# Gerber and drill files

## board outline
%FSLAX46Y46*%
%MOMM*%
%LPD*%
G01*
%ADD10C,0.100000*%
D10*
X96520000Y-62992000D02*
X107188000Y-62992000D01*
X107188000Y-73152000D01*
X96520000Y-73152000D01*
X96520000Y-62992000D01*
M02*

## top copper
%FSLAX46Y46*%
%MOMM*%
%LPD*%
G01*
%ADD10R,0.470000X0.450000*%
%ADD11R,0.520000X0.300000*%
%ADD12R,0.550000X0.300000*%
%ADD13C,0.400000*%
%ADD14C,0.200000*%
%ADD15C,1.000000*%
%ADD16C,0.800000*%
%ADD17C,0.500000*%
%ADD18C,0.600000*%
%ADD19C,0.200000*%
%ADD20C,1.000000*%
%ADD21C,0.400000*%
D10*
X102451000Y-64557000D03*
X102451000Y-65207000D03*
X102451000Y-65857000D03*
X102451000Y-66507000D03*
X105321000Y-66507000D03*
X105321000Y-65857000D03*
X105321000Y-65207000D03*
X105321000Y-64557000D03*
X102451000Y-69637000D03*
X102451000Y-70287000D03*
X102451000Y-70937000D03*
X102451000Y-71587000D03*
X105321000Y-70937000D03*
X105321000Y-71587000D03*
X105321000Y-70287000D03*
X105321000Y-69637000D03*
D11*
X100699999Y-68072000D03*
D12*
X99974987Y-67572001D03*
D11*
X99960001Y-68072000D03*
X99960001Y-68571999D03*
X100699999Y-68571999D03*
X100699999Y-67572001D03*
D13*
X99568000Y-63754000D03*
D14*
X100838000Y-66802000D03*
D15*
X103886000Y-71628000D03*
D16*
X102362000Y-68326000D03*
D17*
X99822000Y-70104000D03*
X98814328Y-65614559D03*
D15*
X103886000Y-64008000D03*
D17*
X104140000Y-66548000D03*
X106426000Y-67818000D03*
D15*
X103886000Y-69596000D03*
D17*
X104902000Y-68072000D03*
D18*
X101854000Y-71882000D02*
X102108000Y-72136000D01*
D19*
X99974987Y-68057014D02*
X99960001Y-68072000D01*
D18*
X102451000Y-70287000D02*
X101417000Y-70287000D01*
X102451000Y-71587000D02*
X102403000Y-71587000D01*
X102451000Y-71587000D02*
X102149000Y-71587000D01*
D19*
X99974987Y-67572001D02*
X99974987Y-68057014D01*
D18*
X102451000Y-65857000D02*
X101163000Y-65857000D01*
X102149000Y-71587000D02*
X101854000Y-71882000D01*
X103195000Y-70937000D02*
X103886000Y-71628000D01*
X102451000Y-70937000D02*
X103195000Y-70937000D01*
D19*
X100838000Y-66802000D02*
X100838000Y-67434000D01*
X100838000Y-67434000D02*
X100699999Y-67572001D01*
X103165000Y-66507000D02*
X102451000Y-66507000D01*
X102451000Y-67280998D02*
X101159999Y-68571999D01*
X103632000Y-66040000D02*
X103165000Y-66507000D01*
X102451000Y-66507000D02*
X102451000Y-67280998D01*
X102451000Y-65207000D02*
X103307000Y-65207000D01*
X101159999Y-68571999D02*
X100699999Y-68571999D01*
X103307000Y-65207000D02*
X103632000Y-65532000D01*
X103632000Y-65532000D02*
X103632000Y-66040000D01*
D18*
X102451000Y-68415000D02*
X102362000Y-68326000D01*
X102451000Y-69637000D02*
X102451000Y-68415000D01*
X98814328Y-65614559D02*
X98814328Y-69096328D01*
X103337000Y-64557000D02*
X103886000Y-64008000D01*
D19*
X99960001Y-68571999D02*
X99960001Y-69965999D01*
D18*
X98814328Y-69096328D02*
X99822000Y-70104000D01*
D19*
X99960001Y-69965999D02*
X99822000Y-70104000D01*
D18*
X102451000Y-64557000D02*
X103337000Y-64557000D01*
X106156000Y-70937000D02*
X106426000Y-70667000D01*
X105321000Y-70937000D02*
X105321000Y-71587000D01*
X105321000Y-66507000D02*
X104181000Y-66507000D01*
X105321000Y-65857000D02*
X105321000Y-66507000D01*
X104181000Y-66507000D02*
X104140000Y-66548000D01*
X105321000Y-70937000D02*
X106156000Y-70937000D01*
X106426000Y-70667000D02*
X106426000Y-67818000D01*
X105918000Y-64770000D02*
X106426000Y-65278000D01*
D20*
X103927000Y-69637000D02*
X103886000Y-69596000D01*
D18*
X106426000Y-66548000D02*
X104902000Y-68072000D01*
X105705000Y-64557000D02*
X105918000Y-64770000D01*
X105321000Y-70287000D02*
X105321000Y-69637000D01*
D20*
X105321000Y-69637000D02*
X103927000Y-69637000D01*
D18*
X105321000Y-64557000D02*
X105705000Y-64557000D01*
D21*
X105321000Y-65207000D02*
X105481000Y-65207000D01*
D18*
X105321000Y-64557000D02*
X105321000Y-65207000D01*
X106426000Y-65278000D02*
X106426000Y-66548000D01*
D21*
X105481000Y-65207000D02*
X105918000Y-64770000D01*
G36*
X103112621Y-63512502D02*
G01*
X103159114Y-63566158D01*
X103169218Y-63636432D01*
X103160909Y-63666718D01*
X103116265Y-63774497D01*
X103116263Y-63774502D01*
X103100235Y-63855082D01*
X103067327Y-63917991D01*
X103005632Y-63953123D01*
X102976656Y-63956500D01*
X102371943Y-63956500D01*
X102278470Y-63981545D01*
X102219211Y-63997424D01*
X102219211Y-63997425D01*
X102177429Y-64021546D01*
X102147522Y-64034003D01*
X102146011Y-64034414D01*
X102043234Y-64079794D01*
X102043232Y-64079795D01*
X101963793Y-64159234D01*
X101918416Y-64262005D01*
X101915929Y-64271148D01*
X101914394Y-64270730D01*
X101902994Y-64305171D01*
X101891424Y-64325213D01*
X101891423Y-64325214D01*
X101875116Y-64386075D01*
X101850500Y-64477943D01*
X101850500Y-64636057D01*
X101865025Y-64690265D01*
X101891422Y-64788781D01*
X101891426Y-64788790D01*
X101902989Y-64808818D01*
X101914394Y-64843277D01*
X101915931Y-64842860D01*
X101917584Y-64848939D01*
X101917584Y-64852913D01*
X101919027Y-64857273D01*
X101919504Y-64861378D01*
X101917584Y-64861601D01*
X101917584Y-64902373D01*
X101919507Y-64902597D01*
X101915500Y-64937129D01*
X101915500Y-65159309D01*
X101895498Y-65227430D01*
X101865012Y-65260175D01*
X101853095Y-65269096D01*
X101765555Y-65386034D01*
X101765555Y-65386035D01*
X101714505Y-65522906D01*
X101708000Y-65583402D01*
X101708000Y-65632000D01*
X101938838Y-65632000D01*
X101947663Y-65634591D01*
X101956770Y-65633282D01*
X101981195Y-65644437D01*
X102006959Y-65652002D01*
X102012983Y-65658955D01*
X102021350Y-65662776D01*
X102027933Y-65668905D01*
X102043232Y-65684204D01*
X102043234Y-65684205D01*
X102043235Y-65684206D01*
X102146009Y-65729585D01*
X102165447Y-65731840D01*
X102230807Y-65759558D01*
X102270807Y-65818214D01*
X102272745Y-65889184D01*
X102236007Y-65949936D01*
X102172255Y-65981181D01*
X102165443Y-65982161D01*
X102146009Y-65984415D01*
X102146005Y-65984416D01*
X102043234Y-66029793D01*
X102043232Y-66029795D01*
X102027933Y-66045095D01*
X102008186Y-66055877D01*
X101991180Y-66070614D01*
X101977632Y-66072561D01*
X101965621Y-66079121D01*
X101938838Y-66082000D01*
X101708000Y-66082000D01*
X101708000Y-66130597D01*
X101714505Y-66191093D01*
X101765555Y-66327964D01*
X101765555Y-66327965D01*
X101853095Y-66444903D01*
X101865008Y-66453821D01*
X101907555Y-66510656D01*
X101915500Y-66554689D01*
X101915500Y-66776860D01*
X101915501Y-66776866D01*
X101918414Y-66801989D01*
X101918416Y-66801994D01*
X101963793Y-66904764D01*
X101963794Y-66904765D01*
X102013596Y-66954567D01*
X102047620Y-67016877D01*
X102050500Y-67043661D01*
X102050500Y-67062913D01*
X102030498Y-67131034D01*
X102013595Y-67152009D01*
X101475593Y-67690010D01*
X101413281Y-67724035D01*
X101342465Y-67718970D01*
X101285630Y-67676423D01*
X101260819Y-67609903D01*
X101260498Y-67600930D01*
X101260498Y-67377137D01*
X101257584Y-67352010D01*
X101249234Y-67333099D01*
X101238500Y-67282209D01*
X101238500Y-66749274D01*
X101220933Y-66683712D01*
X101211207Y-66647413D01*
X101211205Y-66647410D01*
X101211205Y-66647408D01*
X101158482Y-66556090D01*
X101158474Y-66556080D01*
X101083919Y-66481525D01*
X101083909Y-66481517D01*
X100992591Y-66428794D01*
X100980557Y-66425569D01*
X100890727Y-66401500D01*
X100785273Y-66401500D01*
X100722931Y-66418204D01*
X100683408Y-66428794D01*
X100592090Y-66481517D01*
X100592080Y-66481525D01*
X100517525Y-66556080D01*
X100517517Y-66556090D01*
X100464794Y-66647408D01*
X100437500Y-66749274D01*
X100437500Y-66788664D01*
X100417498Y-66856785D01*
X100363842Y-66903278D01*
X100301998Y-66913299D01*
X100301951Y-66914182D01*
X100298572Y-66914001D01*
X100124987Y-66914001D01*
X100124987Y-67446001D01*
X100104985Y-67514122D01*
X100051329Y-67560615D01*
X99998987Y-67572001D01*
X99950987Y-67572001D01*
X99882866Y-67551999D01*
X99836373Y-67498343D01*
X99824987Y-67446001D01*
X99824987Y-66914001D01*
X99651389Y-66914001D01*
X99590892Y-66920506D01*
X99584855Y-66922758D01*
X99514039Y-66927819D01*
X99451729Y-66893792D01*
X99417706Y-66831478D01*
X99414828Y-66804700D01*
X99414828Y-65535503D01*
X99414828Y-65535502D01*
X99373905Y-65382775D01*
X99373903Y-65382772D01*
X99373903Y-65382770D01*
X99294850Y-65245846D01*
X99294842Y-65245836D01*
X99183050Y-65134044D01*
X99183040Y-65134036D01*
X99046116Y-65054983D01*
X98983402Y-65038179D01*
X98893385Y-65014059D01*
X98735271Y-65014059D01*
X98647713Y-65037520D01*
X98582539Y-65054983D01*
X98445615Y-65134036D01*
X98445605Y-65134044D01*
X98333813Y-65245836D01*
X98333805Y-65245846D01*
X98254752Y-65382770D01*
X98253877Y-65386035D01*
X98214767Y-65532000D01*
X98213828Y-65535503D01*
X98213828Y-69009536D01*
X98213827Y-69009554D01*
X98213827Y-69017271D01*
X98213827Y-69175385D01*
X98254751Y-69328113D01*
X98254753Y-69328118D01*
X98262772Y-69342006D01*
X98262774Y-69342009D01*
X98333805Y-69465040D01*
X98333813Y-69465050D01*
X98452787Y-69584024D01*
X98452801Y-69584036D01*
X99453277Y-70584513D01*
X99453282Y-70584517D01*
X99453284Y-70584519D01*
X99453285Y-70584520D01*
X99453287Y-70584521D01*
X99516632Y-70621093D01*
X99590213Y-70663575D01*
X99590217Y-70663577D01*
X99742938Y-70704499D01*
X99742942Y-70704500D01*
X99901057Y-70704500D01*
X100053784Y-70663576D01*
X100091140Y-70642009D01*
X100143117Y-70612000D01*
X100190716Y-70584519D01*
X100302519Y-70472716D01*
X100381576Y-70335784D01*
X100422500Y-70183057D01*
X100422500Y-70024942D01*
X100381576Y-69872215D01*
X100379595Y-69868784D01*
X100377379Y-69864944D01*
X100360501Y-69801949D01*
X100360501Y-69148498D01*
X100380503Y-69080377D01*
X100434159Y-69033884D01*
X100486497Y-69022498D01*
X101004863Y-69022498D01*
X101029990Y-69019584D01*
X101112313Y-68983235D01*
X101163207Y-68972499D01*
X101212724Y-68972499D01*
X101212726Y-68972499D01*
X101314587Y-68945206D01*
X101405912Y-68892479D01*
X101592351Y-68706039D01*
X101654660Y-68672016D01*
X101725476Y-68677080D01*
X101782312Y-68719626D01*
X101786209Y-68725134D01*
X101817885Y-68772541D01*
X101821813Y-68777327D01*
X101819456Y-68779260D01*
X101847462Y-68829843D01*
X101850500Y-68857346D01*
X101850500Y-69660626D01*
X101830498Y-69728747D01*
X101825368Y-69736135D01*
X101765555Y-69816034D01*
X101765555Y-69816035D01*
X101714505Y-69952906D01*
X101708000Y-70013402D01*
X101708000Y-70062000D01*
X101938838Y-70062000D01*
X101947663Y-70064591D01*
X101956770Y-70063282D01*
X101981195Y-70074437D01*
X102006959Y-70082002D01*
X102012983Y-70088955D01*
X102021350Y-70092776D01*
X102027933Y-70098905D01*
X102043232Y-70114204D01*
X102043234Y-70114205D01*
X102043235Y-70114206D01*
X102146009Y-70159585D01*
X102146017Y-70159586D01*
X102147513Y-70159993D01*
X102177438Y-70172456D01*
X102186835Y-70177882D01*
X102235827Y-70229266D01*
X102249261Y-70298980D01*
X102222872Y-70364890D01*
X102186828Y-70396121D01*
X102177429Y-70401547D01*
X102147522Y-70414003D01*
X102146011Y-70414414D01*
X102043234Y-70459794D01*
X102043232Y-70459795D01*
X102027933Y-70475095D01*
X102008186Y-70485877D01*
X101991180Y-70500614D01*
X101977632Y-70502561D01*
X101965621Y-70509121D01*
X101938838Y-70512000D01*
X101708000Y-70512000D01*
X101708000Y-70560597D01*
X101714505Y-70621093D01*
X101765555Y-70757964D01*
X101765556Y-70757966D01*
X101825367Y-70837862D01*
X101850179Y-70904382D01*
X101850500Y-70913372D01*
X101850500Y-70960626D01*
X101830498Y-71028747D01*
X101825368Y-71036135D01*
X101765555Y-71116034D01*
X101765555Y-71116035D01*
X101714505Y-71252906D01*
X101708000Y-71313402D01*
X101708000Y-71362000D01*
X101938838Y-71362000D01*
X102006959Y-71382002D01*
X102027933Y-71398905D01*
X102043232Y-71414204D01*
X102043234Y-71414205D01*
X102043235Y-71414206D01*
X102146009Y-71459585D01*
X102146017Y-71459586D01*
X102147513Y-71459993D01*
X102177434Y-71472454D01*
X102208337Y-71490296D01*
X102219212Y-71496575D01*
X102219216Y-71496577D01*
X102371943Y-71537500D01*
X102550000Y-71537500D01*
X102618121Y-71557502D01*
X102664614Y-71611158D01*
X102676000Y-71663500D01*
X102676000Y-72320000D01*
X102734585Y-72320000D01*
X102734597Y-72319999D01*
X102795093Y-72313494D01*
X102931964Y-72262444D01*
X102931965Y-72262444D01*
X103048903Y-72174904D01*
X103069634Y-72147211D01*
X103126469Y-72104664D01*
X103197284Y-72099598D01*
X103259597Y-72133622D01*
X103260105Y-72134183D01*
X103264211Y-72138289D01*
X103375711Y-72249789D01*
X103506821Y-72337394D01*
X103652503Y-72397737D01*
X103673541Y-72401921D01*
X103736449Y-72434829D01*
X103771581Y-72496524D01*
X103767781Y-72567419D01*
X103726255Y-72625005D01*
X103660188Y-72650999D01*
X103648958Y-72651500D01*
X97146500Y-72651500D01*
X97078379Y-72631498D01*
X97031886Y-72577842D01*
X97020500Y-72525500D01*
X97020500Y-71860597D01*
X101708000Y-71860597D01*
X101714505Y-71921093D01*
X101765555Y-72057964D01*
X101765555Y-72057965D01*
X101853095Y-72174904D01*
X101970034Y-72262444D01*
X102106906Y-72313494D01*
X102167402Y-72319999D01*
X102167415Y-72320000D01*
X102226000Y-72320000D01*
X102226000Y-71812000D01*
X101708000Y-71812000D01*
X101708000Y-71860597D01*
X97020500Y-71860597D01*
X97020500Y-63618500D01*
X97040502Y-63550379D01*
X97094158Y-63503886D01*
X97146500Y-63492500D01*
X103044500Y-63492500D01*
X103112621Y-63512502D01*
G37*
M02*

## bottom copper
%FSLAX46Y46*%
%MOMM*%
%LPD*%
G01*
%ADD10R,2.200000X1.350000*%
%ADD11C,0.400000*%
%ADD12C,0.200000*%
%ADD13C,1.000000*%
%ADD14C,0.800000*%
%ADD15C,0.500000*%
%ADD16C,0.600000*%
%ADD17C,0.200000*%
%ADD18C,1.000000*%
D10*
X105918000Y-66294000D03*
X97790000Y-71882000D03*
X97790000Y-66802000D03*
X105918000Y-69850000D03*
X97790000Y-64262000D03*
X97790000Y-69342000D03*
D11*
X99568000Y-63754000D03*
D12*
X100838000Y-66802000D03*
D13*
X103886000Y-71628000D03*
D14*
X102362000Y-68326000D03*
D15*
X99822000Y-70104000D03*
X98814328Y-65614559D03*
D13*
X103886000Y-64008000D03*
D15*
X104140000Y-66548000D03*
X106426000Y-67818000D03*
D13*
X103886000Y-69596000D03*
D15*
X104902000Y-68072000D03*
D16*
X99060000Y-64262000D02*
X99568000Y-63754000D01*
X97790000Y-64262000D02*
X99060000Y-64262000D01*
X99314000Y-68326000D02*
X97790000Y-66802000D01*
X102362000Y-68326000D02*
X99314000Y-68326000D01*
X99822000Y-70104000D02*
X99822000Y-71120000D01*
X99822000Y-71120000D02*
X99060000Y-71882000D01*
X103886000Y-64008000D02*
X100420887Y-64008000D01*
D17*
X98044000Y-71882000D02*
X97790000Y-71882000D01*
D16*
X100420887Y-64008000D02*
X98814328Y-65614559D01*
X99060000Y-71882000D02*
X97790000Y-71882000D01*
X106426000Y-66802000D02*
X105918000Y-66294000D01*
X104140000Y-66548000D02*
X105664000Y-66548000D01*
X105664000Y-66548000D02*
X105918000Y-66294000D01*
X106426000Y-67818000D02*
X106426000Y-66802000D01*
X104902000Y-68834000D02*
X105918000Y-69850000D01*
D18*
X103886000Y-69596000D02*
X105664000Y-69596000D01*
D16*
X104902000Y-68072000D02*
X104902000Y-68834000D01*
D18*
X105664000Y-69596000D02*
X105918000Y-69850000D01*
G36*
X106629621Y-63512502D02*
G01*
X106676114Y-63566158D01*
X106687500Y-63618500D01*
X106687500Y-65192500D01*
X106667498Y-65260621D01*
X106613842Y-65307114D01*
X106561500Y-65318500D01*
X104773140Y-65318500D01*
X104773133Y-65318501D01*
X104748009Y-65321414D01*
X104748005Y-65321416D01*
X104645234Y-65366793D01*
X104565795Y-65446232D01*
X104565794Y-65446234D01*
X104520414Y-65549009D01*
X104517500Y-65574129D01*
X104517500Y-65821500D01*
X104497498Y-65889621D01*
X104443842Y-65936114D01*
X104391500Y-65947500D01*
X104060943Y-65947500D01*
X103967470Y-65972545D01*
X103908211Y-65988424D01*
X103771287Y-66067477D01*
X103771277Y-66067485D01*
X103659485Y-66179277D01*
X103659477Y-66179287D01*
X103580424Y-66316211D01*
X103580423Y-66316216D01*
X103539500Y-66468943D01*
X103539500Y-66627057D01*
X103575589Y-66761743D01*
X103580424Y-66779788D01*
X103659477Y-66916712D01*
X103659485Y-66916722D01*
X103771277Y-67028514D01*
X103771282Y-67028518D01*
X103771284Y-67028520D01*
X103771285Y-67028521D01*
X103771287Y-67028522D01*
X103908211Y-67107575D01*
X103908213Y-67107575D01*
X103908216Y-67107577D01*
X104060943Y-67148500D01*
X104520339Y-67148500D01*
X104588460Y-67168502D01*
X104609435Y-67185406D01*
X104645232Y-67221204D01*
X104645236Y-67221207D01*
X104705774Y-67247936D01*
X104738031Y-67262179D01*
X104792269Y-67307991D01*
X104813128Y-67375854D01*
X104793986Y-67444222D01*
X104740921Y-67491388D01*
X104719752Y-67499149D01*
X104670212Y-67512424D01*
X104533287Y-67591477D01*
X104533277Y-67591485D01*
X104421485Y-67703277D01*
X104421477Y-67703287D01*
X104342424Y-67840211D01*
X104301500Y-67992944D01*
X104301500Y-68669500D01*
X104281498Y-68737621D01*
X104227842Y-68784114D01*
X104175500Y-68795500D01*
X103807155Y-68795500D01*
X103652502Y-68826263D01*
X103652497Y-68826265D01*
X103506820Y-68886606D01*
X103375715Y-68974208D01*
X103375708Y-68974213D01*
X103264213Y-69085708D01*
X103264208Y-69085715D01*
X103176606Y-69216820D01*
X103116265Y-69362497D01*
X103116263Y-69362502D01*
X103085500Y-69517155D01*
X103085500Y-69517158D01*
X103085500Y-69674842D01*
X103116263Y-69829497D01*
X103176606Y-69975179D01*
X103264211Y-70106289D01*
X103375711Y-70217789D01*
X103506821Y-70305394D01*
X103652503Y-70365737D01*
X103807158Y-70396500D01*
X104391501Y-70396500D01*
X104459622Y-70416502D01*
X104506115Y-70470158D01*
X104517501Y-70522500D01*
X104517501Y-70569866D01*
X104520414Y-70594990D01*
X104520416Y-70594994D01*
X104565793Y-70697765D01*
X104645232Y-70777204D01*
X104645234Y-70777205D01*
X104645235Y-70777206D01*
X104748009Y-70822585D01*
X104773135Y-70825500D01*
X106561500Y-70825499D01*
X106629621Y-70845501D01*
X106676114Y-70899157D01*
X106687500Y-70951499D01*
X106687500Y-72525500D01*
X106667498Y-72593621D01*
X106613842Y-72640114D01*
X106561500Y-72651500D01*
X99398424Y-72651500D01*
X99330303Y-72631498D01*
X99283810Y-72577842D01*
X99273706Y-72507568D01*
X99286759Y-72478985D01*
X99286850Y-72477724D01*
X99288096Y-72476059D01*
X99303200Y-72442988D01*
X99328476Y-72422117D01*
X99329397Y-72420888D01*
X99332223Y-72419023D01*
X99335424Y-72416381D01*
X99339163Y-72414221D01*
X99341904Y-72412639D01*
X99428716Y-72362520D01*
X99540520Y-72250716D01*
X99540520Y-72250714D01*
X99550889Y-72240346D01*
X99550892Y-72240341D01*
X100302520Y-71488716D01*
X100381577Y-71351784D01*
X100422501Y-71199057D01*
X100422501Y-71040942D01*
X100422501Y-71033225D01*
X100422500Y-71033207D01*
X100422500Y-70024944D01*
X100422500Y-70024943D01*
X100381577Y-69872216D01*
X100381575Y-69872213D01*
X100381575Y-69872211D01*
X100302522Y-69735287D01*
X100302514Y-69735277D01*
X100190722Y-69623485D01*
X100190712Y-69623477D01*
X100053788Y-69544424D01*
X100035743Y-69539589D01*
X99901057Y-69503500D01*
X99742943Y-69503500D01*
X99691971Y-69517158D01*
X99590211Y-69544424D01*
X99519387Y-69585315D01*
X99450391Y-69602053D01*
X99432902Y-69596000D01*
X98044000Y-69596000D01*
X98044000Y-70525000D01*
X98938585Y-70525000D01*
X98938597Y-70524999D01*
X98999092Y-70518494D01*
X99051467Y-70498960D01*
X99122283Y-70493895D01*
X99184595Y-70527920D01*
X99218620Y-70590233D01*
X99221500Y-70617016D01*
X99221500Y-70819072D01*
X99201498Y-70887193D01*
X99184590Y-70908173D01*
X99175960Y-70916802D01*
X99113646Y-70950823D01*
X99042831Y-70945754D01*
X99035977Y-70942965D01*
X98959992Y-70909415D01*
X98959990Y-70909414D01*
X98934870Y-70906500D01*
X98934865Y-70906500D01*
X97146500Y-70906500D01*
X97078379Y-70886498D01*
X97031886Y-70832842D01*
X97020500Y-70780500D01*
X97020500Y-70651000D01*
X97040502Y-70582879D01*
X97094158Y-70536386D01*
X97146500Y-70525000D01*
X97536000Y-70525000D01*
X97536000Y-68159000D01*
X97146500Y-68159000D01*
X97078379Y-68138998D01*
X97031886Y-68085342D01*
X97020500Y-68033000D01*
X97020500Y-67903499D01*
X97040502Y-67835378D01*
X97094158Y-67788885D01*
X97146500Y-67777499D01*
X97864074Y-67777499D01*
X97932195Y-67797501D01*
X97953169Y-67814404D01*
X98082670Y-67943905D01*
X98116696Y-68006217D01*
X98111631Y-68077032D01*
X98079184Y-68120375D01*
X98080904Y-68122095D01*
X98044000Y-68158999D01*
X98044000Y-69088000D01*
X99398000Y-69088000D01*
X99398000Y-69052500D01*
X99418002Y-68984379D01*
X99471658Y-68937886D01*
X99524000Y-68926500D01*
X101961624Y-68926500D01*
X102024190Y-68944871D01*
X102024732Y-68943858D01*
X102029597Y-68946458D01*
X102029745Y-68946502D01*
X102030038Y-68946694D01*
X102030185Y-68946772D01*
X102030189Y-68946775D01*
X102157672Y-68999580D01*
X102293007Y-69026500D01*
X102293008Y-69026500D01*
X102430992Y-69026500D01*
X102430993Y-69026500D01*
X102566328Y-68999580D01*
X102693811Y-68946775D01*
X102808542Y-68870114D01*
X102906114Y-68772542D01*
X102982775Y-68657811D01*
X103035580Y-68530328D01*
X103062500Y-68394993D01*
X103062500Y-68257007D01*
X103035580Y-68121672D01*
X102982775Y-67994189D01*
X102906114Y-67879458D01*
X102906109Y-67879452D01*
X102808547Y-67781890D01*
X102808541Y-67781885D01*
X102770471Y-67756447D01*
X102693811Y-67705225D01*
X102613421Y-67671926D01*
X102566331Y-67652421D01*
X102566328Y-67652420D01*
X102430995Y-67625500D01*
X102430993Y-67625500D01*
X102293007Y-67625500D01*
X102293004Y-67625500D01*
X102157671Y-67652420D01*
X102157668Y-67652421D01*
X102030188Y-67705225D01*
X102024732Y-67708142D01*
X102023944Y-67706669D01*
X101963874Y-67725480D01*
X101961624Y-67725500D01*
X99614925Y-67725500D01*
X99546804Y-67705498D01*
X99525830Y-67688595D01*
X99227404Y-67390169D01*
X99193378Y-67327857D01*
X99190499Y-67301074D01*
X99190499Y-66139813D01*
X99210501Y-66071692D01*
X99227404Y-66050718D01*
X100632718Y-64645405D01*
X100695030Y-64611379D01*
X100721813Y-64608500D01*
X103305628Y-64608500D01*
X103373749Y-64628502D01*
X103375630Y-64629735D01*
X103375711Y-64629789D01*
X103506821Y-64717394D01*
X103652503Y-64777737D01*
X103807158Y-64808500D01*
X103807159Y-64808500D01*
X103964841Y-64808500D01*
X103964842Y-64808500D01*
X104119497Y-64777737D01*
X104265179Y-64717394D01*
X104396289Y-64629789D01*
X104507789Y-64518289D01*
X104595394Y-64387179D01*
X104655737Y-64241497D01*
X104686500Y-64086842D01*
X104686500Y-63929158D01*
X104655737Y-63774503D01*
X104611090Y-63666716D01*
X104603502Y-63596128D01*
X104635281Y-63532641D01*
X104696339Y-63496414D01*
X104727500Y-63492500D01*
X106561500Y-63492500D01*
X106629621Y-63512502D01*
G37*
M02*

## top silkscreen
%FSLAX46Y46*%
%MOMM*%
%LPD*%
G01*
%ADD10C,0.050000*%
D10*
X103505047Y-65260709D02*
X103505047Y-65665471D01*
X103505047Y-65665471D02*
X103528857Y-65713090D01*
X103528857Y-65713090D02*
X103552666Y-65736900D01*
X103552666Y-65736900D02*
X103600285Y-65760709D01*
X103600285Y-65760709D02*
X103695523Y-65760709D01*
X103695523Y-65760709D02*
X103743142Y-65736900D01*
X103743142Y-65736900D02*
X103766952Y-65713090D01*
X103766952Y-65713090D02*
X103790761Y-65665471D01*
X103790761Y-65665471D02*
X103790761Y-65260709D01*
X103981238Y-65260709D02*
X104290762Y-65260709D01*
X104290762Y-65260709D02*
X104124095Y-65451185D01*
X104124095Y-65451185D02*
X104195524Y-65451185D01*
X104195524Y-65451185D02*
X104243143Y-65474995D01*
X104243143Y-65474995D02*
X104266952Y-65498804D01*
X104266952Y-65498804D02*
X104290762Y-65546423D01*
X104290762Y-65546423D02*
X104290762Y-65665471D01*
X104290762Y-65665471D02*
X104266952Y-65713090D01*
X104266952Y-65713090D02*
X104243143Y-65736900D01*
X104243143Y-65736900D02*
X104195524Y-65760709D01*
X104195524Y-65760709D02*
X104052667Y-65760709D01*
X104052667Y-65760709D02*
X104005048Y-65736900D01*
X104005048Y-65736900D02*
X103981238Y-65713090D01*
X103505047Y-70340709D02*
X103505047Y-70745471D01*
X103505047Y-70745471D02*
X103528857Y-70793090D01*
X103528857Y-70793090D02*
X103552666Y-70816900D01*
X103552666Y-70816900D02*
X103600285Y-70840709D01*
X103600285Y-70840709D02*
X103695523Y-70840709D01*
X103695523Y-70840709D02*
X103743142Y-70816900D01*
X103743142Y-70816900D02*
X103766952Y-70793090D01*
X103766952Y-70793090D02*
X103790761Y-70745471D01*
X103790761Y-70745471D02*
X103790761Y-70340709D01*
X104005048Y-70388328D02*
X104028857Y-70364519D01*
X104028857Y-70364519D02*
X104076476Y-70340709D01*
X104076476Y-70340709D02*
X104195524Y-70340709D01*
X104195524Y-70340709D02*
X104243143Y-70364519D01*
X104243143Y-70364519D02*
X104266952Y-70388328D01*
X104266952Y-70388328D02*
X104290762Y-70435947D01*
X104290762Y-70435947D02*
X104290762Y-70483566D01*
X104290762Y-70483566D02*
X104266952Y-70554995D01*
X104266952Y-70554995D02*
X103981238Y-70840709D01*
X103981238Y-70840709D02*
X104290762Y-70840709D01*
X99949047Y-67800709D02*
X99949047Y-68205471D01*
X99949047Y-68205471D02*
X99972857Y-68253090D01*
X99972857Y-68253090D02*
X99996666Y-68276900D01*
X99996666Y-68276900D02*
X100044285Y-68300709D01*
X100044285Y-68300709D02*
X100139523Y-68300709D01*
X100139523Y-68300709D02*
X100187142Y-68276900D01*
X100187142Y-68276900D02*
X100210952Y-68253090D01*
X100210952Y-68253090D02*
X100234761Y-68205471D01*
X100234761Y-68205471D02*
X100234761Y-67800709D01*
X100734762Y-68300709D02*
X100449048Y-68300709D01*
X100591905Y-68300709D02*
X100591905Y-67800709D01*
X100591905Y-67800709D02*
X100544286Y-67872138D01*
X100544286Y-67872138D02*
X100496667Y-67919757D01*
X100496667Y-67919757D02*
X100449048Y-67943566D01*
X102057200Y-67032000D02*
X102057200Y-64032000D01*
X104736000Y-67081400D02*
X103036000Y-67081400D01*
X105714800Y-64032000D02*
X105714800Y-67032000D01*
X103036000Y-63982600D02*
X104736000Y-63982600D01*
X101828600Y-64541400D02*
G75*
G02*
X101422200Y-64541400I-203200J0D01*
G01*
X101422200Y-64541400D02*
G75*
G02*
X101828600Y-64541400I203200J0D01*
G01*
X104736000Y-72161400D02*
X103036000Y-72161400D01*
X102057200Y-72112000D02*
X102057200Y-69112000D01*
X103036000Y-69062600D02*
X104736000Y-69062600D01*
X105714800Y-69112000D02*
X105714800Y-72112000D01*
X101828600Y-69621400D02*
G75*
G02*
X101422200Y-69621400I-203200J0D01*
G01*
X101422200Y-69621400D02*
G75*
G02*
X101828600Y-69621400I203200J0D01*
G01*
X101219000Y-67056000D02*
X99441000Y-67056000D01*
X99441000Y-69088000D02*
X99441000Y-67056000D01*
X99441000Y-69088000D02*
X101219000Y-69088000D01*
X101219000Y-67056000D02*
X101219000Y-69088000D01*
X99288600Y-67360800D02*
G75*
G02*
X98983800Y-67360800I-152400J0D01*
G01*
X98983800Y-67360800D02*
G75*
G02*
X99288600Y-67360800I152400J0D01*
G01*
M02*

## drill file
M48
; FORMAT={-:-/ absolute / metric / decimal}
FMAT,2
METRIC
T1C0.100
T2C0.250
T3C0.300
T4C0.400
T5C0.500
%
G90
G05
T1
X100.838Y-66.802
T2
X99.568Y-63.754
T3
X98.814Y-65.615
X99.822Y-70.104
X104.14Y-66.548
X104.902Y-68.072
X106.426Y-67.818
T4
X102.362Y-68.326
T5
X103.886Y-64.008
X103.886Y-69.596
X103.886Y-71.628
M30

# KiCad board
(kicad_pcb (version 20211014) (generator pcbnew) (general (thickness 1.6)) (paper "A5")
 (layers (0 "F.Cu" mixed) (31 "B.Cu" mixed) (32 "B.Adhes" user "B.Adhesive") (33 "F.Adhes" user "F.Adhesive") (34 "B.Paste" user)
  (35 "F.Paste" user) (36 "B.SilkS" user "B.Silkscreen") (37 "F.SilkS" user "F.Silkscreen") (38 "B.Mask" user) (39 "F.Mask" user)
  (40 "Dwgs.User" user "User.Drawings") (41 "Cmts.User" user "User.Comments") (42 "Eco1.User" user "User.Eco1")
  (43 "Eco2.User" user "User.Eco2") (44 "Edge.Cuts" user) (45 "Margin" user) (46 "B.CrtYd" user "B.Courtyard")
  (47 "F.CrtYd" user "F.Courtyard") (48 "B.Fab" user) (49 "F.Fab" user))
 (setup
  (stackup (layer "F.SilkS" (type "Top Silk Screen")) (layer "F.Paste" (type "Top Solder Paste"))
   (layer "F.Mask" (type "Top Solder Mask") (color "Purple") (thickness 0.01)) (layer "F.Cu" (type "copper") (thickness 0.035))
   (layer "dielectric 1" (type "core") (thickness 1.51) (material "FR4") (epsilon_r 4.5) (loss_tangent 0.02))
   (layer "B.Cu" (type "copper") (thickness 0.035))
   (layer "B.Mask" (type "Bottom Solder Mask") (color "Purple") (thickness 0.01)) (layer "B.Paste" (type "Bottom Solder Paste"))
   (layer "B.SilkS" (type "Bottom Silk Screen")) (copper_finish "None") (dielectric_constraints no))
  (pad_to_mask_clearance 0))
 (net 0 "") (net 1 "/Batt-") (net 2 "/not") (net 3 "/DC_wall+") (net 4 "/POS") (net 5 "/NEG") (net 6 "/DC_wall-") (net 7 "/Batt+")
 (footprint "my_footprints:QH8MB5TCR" (layer "F.Cu") (at 103.886 65.532)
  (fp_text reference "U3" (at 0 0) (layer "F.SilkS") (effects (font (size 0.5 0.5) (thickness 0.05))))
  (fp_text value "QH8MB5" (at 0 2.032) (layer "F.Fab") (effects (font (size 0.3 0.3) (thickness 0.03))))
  (fp_line (start -1.8288 1.5) (end -1.8288 -1.5) (layer "F.SilkS") (width 0.05))
  (fp_line (start 0.85 1.5494) (end -0.85 1.5494) (layer "F.SilkS") (width 0.05))
  (fp_line (start 1.8288 -1.5) (end 1.8288 1.5) (layer "F.SilkS") (width 0.05))
  (fp_line (start -0.85 -1.5494) (end 0.85 -1.5494) (layer "F.SilkS") (width 0.05))
  (fp_circle (center -2.2606 -0.9906) (end -2.0574 -0.9906) (layer "F.SilkS") (width 0.05) (fill none))
  (pad "1" smd rect (at -1.435 -0.975 90) (size 0.45 0.47) (layers "F.Cu" "F.Paste" "F.Mask") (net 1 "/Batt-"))
  (pad "2" smd rect (at -1.435 -0.325 90) (size 0.45 0.47) (layers "F.Cu" "F.Paste" "F.Mask") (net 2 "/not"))
  (pad "3" smd rect (at -1.435 0.325 90) (size 0.45 0.47) (layers "F.Cu" "F.Paste" "F.Mask") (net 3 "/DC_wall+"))
  (pad "4" smd rect (at -1.435 0.975 90) (size 0.45 0.47) (layers "F.Cu" "F.Paste" "F.Mask") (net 2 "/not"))
  (pad "5" smd rect (at 1.435 0.975 90) (size 0.45 0.47) (layers "F.Cu" "F.Paste" "F.Mask") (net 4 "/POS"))
  (pad "5" smd rect (at 1.435 0.325 90) (size 0.45 0.47) (layers "F.Cu" "F.Paste" "F.Mask") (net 4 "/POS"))
  (pad "6" smd rect (at 1.435 -0.325 90) (size 0.45 0.47) (layers "F.Cu" "F.Paste" "F.Mask") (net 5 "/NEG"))
  (pad "6" smd rect (at 1.435 -0.975 90) (size 0.45 0.47) (layers "F.Cu" "F.Paste" "F.Mask") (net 5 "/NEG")))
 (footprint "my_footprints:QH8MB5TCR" (layer "F.Cu") (at 103.886 70.612)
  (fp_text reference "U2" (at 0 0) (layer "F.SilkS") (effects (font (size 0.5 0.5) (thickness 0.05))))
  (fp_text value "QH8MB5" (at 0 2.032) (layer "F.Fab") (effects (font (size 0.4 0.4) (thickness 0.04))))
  (fp_line (start 0.85 1.5494) (end -0.85 1.5494) (layer "F.SilkS") (width 0.05))
  (fp_line (start -1.8288 1.5) (end -1.8288 -1.5) (layer "F.SilkS") (width 0.05))
  (fp_line (start -0.85 -1.5494) (end 0.85 -1.5494) (layer "F.SilkS") (width 0.05))
  (fp_line (start 1.8288 -1.5) (end 1.8288 1.5) (layer "F.SilkS") (width 0.05))
  (fp_circle (center -2.2606 -0.9906) (end -2.0574 -0.9906) (layer "F.SilkS") (width 0.05) (fill none))
  (pad "1" smd rect (at -1.435 -0.975 90) (size 0.45 0.47) (layers "F.Cu" "F.Paste" "F.Mask") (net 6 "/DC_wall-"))
  (pad "2" smd rect (at -1.435 -0.325 90) (size 0.45 0.47) (layers "F.Cu" "F.Paste" "F.Mask") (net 3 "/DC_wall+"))
  (pad "3" smd rect (at -1.435 0.325 90) (size 0.45 0.47) (layers "F.Cu" "F.Paste" "F.Mask") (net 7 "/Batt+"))
  (pad "4" smd rect (at -1.435 0.975 90) (size 0.45 0.47) (layers "F.Cu" "F.Paste" "F.Mask") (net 3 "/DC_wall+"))
  (pad "5" smd rect (at 1.435 0.325 90) (size 0.45 0.47) (layers "F.Cu" "F.Paste" "F.Mask") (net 4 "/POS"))
  (pad "5" smd rect (at 1.435 0.975 90) (size 0.45 0.47) (layers "F.Cu" "F.Paste" "F.Mask") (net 4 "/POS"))
  (pad "6" smd rect (at 1.435 -0.325 90) (size 0.45 0.47) (layers "F.Cu" "F.Paste" "F.Mask") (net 5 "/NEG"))
  (pad "6" smd rect (at 1.435 -0.975 90) (size 0.45 0.47) (layers "F.Cu" "F.Paste" "F.Mask") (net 5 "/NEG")))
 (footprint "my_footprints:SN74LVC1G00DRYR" (layer "F.Cu") (at 100.33 68.072)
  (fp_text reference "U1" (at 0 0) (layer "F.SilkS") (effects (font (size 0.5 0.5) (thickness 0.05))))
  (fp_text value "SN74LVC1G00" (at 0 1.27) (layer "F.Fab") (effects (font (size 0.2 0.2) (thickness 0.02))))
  (fp_line (start 0.889 -1.016) (end -0.889 -1.016) (layer "F.SilkS") (width 0.05))
  (fp_line (start -0.889 1.016) (end -0.889 -1.016) (layer "F.SilkS") (width 0.05))
  (fp_line (start -0.889 1.016) (end 0.889 1.016) (layer "F.SilkS") (width 0.05))
  (fp_line (start 0.889 -1.016) (end 0.889 1.016) (layer "F.SilkS") (width 0.05))
  (fp_circle (center -1.1938 -0.7112) (end -1.0414 -0.7112) (layer "F.SilkS") (width 0.05) (fill none))
  (pad "" smd rect (at 0.369999 0) (size 0.52 0.3) (layers "F.Cu" "F.Mask"))
  (pad "1" smd rect (at -0.355013 -0.499999) (size 0.55 0.3) (layers "F.Cu" "F.Mask") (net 3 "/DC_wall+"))
  (pad "2" smd rect (at -0.369999 0) (size 0.52 0.3) (layers "F.Cu" "F.Mask") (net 3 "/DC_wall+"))
  (pad "3" smd rect (at -0.369999 0.499999) (size 0.52 0.3) (layers "F.Cu" "F.Mask") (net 1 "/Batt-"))
  (pad "4" smd rect (at 0.369999 0.499999) (size 0.52 0.3) (layers "F.Cu" "F.Mask") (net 2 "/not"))
  (pad "5" smd rect (at 0.369999 -0.499999) (size 0.52 0.3) (layers "F.Cu" "F.Mask") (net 7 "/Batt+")))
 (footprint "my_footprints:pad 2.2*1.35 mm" (layer "B.Cu") (at 105.918 66.294 180)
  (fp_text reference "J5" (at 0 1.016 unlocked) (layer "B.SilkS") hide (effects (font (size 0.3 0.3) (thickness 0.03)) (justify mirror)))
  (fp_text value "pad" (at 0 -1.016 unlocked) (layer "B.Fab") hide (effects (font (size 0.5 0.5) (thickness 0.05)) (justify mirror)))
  (pad "1" smd rect (at 0 0 180) (size 2.2 1.35) (layers "B.Cu" "B.Paste" "B.Mask") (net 4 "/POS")))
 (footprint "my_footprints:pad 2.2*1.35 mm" (layer "B.Cu") (at 97.79 71.882 180)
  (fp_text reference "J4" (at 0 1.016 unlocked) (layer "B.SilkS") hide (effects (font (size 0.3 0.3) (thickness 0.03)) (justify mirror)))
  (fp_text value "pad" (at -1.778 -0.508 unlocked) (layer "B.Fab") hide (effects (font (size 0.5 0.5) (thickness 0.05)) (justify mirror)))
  (pad "1" smd rect (at 0 0 180) (size 2.2 1.35) (layers "B.Cu" "B.Paste" "B.Mask") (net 1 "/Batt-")))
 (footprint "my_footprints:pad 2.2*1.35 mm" (layer "B.Cu") (at 97.79 66.802)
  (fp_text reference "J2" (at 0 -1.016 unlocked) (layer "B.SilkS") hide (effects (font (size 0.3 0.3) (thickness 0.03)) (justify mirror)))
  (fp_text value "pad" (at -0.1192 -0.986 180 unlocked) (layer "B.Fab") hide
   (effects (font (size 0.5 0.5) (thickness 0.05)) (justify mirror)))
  (pad "1" smd rect (at 0 0) (size 2.2 1.35) (layers "B.Cu" "B.Paste" "B.Mask") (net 6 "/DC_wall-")))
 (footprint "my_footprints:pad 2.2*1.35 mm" (layer "B.Cu") (at 105.918 69.85 180)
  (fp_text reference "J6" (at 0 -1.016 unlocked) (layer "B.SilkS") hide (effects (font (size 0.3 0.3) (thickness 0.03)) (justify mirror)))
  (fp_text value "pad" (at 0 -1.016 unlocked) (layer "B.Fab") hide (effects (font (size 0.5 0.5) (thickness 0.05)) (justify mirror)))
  (pad "1" smd rect (at 0 0 180) (size 2.2 1.35) (layers "B.Cu" "B.Paste" "B.Mask") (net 5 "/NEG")))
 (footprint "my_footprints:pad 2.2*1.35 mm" (layer "B.Cu") (at 97.79 64.262 180)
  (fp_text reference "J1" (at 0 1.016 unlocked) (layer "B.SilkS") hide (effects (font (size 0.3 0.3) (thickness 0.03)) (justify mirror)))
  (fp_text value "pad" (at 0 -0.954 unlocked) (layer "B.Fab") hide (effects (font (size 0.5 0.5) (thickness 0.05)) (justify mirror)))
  (pad "1" smd rect (at 0 0 180) (size 2.2 1.35) (layers "B.Cu" "B.Paste" "B.Mask") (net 3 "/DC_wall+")))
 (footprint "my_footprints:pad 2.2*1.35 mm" (layer "B.Cu") (at 97.79 69.342 180)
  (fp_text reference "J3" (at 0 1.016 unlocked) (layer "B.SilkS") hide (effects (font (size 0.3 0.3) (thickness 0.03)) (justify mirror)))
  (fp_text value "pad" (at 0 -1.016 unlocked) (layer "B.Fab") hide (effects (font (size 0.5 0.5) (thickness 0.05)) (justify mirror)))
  (pad "1" smd rect (at 0 0 180) (size 2.2 1.35) (layers "B.Cu" "B.Paste" "B.Mask") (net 7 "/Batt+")))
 (gr_rect (start 96.52 62.992) (end 107.188 73.152) (layer "Edge.Cuts") (width 0.1) (fill none))
 (segment (start 101.854 71.882) (end 102.108 72.136) (width 0.6) (layer "F.Cu") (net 3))
 (segment (start 99.974987 68.057014) (end 99.960001 68.072) (width 0.2) (layer "F.Cu") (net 3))
 (segment (start 102.451 70.287) (end 101.417 70.287) (width 0.6) (layer "F.Cu") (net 3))
 (segment (start 102.451 71.587) (end 102.403 71.587) (width 0.6) (layer "F.Cu") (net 3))
 (segment (start 102.451 71.587) (end 102.149 71.587) (width 0.6) (layer "F.Cu") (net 3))
 (segment (start 99.974987 67.572001) (end 99.974987 68.057014) (width 0.2) (layer "F.Cu") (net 3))
 (segment (start 102.451 65.857) (end 101.163 65.857) (width 0.6) (layer "F.Cu") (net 3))
 (segment (start 102.149 71.587) (end 101.854 71.882) (width 0.6) (layer "F.Cu") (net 3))
 (via (at 99.568 63.754) (size 0.4) (drill 0.25) (layers "F.Cu" "B.Cu") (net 3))
 (segment (start 99.06 64.262) (end 99.568 63.754) (width 0.6) (layer "B.Cu") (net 3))
 (segment (start 97.79 64.262) (end 99.06 64.262) (width 0.6) (layer "B.Cu") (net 3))
 (segment (start 103.195 70.937) (end 103.886 71.628) (width 0.6) (layer "F.Cu") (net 7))
 (segment (start 102.451 70.937) (end 103.195 70.937) (width 0.6) (layer "F.Cu") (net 7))
 (segment (start 100.838 66.802) (end 100.838 67.434) (width 0.2) (layer "F.Cu") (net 7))
 (segment (start 100.838 67.434) (end 100.699999 67.572001) (width 0.2) (layer "F.Cu") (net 7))
 (via (at 100.838 66.802) (size 0.2) (drill 0.1) (layers "F.Cu" "B.Cu") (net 7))
 (via (at 103.886 71.628) (size 1) (drill 0.5) (layers "F.Cu" "B.Cu") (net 7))
 (segment (start 103.165 66.507) (end 102.451 66.507) (width 0.2) (layer "F.Cu") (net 2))
 (segment (start 102.451 67.280998) (end 101.159999 68.571999) (width 0.2) (layer "F.Cu") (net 2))
 (segment (start 103.632 66.04) (end 103.165 66.507) (width 0.2) (layer "F.Cu") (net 2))
 (segment (start 102.451 66.507) (end 102.451 67.280998) (width 0.2) (layer "F.Cu") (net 2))
 (segment (start 102.451 65.207) (end 103.307 65.207) (width 0.2) (layer "F.Cu") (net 2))
 (segment (start 101.159999 68.571999) (end 100.699999 68.571999) (width 0.2) (layer "F.Cu") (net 2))
 (segment (start 103.307 65.207) (end 103.632 65.532) (width 0.2) (layer "F.Cu") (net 2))
 (segment (start 103.632 65.532) (end 103.632 66.04) (width 0.2) (layer "F.Cu") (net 2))
 (segment (start 102.451 68.415) (end 102.362 68.326) (width 0.6) (layer "F.Cu") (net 6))
 (segment (start 102.451 69.637) (end 102.451 68.415) (width 0.6) (layer "F.Cu") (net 6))
 (via (at 102.362 68.326) (size 0.8) (drill 0.4) (layers "F.Cu" "B.Cu") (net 6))
 (segment (start 99.314 68.326) (end 97.79 66.802) (width 0.6) (layer "B.Cu") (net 6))
 (segment (start 102.362 68.326) (end 99.314 68.326) (width 0.6) (layer "B.Cu") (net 6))
 (segment (start 98.814328 65.614559) (end 98.814328 69.096328) (width 0.6) (layer "F.Cu") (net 1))
 (segment (start 103.337 64.557) (end 103.886 64.008) (width 0.6) (layer "F.Cu") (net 1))
 (segment (start 99.960001 68.571999) (end 99.960001 69.965999) (width 0.2) (layer "F.Cu") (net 1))
 (segment (start 98.814328 69.096328) (end 99.822 70.104) (width 0.6) (layer "F.Cu") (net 1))
 (segment (start 99.960001 69.965999) (end 99.822 70.104) (width 0.2) (layer "F.Cu") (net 1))
 (segment (start 102.451 64.557) (end 103.337 64.557) (width 0.6) (layer "F.Cu") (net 1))
 (via (at 99.822 70.104) (size 0.5) (drill 0.3) (layers "F.Cu" "B.Cu") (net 1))
 (via (at 98.814328 65.614559) (size 0.5) (drill 0.3) (layers "F.Cu" "B.Cu") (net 1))
 (via (at 103.886 64.008) (size 1) (drill 0.5) (layers "F.Cu" "B.Cu") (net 1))
 (segment (start 99.822 70.104) (end 99.822 71.12) (width 0.6) (layer "B.Cu") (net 1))
 (segment (start 99.822 71.12) (end 99.06 71.882) (width 0.6) (layer "B.Cu") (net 1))
 (segment (start 103.886 64.008) (end 100.420887 64.008) (width 0.6) (layer "B.Cu") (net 1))
 (segment (start 98.044 71.882) (end 97.79 71.882) (width 0.2) (layer "B.Cu") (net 1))
 (segment (start 100.420887 64.008) (end 98.814328 65.614559) (width 0.6) (layer "B.Cu") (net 1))
 (segment (start 99.06 71.882) (end 97.79 71.882) (width 0.6) (layer "B.Cu") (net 1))
 (segment (start 106.156 70.937) (end 106.426 70.667) (width 0.6) (layer "F.Cu") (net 4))
 (segment (start 105.321 70.937) (end 105.321 71.587) (width 0.6) (layer "F.Cu") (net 4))
 (segment (start 105.321 66.507) (end 104.181 66.507) (width 0.6) (layer "F.Cu") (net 4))
 (segment (start 105.321 65.857) (end 105.321 66.507) (width 0.6) (layer "F.Cu") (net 4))
 (segment (start 104.181 66.507) (end 104.14 66.548) (width 0.6) (layer "F.Cu") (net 4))
 (segment (start 105.321 70.937) (end 106.156 70.937) (width 0.6) (layer "F.Cu") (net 4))
 (segment (start 106.426 70.667) (end 106.426 67.818) (width 0.6) (layer "F.Cu") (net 4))
 (via (at 104.14 66.548) (size 0.5) (drill 0.3) (layers "F.Cu" "B.Cu") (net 4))
 (via (at 106.426 67.818) (size 0.5) (drill 0.3) (layers "F.Cu" "B.Cu") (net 4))
 (segment (start 106.426 66.802) (end 105.918 66.294) (width 0.6) (layer "B.Cu") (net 4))
 (segment (start 104.14 66.548) (end 105.664 66.548) (width 0.6) (layer "B.Cu") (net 4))
 (segment (start 105.664 66.548) (end 105.918 66.294) (width 0.6) (layer "B.Cu") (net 4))
 (segment (start 106.426 67.818) (end 106.426 66.802) (width 0.6) (layer "B.Cu") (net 4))
 (segment (start 105.918 64.77) (end 106.426 65.278) (width 0.6) (layer "F.Cu") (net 5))
 (segment (start 103.927 69.637) (end 103.886 69.596) (width 1) (layer "F.Cu") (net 5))
 (segment (start 106.426 66.548) (end 104.902 68.072) (width 0.6) (layer "F.Cu") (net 5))
 (segment (start 105.705 64.557) (end 105.918 64.77) (width 0.6) (layer "F.Cu") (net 5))
 (segment (start 105.321 70.287) (end 105.321 69.637) (width 0.6) (layer "F.Cu") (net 5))
 (segment (start 105.321 69.637) (end 103.927 69.637) (width 1) (layer "F.Cu") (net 5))
 (segment (start 105.321 64.557) (end 105.705 64.557) (width 0.6) (layer "F.Cu") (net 5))
 (segment (start 105.321 65.207) (end 105.481 65.207) (width 0.4) (layer "F.Cu") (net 5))
 (segment (start 105.321 64.557) (end 105.321 65.207) (width 0.6) (layer "F.Cu") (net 5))
 (segment (start 106.426 65.278) (end 106.426 66.548) (width 0.6) (layer "F.Cu") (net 5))
 (segment (start 105.481 65.207) (end 105.918 64.77) (width 0.4) (layer "F.Cu") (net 5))
 (via (at 103.886 69.596) (size 1) (drill 0.5) (layers "F.Cu" "B.Cu") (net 5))
 (via (at 104.902 68.072) (size 0.5) (drill 0.3) (layers "F.Cu" "B.Cu") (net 5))
 (segment (start 104.902 68.834) (end 105.918 69.85) (width 0.6) (layer "B.Cu") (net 5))
 (segment (start 103.886 69.596) (end 105.664 69.596) (width 1) (layer "B.Cu") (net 5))
 (segment (start 104.902 68.072) (end 104.902 68.834) (width 0.6) (layer "B.Cu") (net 5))
 (segment (start 105.664 69.596) (end 105.918 69.85) (width 1) (layer "B.Cu") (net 5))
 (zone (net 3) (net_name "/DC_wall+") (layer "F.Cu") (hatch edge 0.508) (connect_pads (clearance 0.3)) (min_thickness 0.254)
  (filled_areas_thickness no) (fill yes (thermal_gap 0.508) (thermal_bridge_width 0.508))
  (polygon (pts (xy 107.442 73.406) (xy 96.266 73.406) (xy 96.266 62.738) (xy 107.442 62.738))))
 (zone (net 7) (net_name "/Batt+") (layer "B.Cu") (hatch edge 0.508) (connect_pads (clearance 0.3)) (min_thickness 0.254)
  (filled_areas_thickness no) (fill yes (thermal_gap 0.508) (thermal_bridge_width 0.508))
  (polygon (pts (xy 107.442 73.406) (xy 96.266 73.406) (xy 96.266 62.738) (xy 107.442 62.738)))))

